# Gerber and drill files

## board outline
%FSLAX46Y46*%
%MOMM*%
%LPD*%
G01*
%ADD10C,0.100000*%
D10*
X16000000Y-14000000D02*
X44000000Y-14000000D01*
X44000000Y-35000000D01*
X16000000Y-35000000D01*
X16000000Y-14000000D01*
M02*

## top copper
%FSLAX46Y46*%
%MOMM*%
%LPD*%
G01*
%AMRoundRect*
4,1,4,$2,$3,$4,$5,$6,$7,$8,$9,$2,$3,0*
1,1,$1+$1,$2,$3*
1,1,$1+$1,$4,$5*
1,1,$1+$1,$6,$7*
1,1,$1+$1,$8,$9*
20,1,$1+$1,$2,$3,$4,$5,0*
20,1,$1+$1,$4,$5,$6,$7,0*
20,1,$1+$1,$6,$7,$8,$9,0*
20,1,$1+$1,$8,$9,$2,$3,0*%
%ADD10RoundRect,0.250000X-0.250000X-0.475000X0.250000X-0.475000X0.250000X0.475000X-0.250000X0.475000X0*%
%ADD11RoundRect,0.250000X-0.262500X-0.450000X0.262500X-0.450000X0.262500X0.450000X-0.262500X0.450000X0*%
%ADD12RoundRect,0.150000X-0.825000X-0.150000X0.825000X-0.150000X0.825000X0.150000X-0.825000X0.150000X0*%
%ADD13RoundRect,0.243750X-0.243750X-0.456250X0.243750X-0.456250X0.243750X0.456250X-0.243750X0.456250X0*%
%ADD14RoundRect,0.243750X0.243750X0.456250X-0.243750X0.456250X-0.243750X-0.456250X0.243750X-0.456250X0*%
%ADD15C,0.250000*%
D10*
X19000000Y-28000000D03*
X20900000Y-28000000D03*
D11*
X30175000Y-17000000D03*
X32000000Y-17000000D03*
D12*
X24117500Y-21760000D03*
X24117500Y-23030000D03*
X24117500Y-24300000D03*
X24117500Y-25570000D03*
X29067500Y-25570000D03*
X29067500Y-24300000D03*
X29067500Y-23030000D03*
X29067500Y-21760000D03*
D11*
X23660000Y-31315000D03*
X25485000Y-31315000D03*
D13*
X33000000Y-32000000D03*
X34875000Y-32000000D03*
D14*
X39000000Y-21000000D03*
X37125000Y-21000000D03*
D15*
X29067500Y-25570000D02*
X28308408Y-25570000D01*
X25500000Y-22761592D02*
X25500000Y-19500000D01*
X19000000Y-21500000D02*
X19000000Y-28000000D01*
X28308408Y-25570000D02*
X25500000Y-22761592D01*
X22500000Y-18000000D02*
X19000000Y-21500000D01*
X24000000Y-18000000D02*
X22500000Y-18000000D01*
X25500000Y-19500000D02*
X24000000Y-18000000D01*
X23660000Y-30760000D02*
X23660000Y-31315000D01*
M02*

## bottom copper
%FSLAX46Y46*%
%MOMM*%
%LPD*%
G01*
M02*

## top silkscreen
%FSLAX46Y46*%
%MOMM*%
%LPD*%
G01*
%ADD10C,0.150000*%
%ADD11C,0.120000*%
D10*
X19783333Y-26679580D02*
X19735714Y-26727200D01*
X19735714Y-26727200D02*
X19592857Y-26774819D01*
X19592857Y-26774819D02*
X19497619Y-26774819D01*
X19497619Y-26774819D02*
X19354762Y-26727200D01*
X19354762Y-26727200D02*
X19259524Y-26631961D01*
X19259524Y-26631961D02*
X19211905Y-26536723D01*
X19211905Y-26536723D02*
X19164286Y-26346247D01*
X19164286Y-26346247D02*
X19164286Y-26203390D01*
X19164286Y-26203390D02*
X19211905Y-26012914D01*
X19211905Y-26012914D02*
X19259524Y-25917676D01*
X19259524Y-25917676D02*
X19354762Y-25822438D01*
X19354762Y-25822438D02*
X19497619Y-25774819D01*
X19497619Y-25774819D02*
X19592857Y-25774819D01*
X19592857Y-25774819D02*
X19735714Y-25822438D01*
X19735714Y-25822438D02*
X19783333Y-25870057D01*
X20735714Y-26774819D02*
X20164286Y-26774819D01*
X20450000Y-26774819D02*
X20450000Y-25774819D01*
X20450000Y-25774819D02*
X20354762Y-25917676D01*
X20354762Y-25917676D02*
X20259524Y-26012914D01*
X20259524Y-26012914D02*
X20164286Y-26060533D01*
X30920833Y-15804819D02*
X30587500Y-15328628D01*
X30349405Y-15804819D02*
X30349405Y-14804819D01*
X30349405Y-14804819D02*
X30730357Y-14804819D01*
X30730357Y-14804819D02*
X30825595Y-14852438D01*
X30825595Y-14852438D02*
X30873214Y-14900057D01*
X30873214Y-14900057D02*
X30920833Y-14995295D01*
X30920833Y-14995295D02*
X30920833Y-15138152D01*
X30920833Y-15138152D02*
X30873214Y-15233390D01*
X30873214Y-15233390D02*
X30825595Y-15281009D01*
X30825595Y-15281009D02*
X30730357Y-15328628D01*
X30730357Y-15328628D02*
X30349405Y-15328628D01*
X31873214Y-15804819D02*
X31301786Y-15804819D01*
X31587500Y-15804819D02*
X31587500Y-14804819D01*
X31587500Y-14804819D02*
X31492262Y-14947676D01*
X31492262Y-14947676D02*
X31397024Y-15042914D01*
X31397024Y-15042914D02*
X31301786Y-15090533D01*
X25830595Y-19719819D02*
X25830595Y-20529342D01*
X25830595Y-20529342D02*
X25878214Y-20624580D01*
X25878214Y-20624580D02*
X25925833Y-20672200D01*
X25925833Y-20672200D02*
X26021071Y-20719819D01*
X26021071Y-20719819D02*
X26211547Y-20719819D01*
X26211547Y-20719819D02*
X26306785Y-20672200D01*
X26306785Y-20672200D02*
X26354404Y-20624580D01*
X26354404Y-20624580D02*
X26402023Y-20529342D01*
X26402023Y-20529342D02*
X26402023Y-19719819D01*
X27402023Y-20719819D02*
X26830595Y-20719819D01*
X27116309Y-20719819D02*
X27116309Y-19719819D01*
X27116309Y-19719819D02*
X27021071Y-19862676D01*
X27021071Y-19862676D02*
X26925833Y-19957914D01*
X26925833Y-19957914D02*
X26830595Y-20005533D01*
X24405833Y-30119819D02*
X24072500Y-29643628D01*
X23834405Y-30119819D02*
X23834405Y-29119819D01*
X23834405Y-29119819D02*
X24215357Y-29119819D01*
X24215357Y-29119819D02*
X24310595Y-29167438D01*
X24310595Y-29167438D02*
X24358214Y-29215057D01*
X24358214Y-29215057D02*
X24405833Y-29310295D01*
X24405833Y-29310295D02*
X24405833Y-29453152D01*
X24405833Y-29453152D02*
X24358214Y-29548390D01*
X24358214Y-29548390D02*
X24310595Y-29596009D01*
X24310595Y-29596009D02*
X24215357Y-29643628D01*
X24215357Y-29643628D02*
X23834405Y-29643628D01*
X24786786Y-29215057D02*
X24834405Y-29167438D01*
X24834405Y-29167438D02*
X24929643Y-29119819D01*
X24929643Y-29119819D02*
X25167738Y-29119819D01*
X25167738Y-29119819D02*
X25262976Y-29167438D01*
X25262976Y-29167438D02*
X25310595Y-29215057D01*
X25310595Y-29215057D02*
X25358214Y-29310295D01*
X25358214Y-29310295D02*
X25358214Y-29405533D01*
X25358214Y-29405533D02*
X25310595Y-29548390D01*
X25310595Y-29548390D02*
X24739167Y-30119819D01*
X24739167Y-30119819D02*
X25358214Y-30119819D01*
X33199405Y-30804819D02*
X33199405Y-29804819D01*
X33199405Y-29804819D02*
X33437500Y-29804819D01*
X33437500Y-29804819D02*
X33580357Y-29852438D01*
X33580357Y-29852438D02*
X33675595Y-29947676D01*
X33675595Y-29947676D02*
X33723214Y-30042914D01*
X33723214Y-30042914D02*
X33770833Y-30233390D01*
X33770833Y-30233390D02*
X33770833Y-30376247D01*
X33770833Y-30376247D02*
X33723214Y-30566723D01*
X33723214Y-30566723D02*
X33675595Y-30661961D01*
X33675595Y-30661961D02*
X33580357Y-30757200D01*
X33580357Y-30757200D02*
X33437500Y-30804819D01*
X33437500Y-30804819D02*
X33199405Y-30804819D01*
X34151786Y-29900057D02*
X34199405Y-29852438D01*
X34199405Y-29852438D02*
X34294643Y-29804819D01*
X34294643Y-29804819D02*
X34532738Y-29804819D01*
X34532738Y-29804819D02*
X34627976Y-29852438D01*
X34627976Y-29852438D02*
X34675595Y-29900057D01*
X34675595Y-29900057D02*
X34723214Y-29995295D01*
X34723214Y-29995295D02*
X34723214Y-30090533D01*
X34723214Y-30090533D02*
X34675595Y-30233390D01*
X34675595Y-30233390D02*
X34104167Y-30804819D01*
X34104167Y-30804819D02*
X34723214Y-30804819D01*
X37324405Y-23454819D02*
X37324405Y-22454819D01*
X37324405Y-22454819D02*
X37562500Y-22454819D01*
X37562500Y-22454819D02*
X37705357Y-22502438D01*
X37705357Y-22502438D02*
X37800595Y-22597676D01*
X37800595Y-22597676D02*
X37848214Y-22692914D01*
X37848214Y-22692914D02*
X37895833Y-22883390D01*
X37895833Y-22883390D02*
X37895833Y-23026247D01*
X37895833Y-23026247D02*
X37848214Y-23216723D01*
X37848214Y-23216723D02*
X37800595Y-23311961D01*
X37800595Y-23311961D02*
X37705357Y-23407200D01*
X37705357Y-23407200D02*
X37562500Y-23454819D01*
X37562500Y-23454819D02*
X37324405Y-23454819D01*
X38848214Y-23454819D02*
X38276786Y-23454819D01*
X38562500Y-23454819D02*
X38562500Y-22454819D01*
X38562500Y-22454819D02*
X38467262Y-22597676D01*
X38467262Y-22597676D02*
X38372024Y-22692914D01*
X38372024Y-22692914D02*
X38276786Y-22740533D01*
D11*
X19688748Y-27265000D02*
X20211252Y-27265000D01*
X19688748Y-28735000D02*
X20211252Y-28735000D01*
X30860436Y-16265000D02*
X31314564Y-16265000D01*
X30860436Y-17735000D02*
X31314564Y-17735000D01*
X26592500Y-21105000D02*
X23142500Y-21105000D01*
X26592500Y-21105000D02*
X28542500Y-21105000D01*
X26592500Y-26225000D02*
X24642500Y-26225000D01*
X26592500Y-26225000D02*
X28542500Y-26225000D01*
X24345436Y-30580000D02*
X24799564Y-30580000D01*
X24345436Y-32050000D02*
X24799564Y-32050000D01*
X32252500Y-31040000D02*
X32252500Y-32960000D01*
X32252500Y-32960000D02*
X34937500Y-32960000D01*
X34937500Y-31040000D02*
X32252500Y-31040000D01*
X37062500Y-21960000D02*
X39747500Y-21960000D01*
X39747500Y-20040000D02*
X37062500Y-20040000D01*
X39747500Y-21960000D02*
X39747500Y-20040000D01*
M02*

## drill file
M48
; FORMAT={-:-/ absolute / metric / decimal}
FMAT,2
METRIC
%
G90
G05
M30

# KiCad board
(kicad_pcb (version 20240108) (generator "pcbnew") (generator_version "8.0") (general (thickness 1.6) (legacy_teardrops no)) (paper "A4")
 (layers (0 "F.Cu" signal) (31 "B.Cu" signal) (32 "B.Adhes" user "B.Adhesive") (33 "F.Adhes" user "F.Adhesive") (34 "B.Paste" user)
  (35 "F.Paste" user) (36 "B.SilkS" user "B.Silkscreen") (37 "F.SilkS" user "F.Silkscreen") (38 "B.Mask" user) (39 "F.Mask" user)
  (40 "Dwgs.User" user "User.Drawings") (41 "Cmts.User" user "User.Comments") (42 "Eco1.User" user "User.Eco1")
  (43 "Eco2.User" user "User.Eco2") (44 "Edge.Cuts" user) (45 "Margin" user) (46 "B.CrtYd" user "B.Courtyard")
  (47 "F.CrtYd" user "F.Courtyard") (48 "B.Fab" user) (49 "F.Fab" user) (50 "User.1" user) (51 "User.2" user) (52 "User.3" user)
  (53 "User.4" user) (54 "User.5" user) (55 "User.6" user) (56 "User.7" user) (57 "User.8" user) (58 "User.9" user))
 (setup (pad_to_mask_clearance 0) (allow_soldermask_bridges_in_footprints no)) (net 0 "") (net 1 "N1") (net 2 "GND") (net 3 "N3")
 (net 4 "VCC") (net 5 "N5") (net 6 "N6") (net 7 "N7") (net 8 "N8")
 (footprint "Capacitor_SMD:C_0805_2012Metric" (layer "F.Cu") (at 19.95 28)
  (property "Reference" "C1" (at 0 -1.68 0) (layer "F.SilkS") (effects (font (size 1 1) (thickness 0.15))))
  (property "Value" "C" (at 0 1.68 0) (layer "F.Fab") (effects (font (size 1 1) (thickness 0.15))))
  (fp_line (start -0.261252 -0.735) (end 0.261252 -0.735) (stroke (width 0.12) (type solid)) (layer "F.SilkS"))
  (fp_line (start -0.261252 0.735) (end 0.261252 0.735) (stroke (width 0.12) (type solid)) (layer "F.SilkS"))
  (pad "1" smd roundrect (at -0.95 0) (size 1 1.45) (layers "F.Cu" "F.Paste" "F.Mask") (roundrect_rratio 0.25) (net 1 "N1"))
  (pad "2" smd roundrect (at 0.95 0) (size 1 1.45) (layers "F.Cu" "F.Paste" "F.Mask") (roundrect_rratio 0.25) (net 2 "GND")))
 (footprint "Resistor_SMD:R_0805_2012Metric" (layer "F.Cu") (at 31.0875 17)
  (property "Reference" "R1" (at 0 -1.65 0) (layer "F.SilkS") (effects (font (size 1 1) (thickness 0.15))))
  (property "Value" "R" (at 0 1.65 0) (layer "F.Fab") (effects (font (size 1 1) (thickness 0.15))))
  (fp_line (start -0.227064 -0.735) (end 0.227064 -0.735) (stroke (width 0.12) (type solid)) (layer "F.SilkS"))
  (fp_line (start -0.227064 0.735) (end 0.227064 0.735) (stroke (width 0.12) (type solid)) (layer "F.SilkS"))
  (pad "1" smd roundrect (at -0.9125 0) (size 1.025 1.4) (layers "F.Cu" "F.Paste" "F.Mask") (roundrect_rratio 0.243902) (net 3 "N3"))
  (pad "2" smd roundrect (at 0.9125 0) (size 1.025 1.4) (layers "F.Cu" "F.Paste" "F.Mask") (roundrect_rratio 0.243902) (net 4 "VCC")))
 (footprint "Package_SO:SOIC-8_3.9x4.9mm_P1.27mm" (layer "F.Cu") (at 26.5925 23.665)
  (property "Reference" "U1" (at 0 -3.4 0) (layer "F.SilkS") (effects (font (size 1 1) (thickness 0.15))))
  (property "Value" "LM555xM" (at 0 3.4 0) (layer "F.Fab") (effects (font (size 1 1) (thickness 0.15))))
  (fp_line (start 0 -2.56) (end -3.45 -2.56) (stroke (width 0.12) (type solid)) (layer "F.SilkS"))
  (fp_line (start 0 -2.56) (end 1.95 -2.56) (stroke (width 0.12) (type solid)) (layer "F.SilkS"))
  (fp_line (start 0 2.56) (end -1.95 2.56) (stroke (width 0.12) (type solid)) (layer "F.SilkS"))
  (fp_line (start 0 2.56) (end 1.95 2.56) (stroke (width 0.12) (type solid)) (layer "F.SilkS"))
  (pad "1" smd roundrect (at -2.475 -1.905) (size 1.95 0.6) (layers "F.Cu" "F.Paste" "F.Mask") (roundrect_rratio 0.25) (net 2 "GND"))
  (pad "2" smd roundrect (at -2.475 -0.635) (size 1.95 0.6) (layers "F.Cu" "F.Paste" "F.Mask") (roundrect_rratio 0.25) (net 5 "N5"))
  (pad "3" smd roundrect (at -2.475 0.635) (size 1.95 0.6) (layers "F.Cu" "F.Paste" "F.Mask") (roundrect_rratio 0.25) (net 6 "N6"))
  (pad "4" smd roundrect (at -2.475 1.905) (size 1.95 0.6) (layers "F.Cu" "F.Paste" "F.Mask") (roundrect_rratio 0.25) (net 4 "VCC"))
  (pad "5" smd roundrect (at 2.475 1.905) (size 1.95 0.6) (layers "F.Cu" "F.Paste" "F.Mask") (roundrect_rratio 0.25) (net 1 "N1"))
  (pad "6" smd roundrect (at 2.475 0.635) (size 1.95 0.6) (layers "F.Cu" "F.Paste" "F.Mask") (roundrect_rratio 0.25) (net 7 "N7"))
  (pad "7" smd roundrect (at 2.475 -0.635) (size 1.95 0.6) (layers "F.Cu" "F.Paste" "F.Mask") (roundrect_rratio 0.25) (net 7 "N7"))
  (pad "8" smd roundrect (at 2.475 -1.905) (size 1.95 0.6) (layers "F.Cu" "F.Paste" "F.Mask") (roundrect_rratio 0.25) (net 4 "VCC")))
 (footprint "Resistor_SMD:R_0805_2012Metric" (layer "F.Cu") (at 24.5725 31.315)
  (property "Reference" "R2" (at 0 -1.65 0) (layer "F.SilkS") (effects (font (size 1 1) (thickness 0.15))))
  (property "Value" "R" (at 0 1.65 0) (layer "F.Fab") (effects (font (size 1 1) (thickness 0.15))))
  (fp_line (start -0.227064 -0.735) (end 0.227064 -0.735) (stroke (width 0.12) (type solid)) (layer "F.SilkS"))
  (fp_line (start -0.227064 0.735) (end 0.227064 0.735) (stroke (width 0.12) (type solid)) (layer "F.SilkS"))
  (pad "1" smd roundrect (at -0.9125 0) (size 1.025 1.4) (layers "F.Cu" "F.Paste" "F.Mask") (roundrect_rratio 0.243902) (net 2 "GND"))
  (pad "2" smd roundrect (at 0.9125 0) (size 1.025 1.4) (layers "F.Cu" "F.Paste" "F.Mask") (roundrect_rratio 0.243902) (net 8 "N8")))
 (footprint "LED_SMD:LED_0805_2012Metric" (layer "F.Cu") (at 33.9375 32)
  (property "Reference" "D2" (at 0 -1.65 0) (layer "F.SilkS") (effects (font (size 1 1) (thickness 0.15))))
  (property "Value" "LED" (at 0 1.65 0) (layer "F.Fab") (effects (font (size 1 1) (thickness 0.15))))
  (fp_line (start -1.685 -0.96) (end -1.685 0.96) (stroke (width 0.12) (type solid)) (layer "F.SilkS"))
  (fp_line (start -1.685 0.96) (end 1 0.96) (stroke (width 0.12) (type solid)) (layer "F.SilkS"))
  (fp_line (start 1 -0.96) (end -1.685 -0.96) (stroke (width 0.12) (type solid)) (layer "F.SilkS"))
  (pad "1" smd roundrect (at -0.9375 0) (size 0.975 1.4) (layers "F.Cu" "F.Paste" "F.Mask") (roundrect_rratio 0.25) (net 8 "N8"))
  (pad "2" smd roundrect (at 0.9375 0) (size 0.975 1.4) (layers "F.Cu" "F.Paste" "F.Mask") (roundrect_rratio 0.25) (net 6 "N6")))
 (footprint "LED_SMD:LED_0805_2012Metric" (layer "F.Cu") (at 38.0625 21 180)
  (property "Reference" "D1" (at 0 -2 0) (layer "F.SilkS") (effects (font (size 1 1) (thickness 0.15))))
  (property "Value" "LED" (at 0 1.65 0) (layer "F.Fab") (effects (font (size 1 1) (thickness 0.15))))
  (fp_line (start 1 -0.96) (end -1.685 -0.96) (stroke (width 0.12) (type solid)) (layer "F.SilkS"))
  (fp_line (start -1.685 0.96) (end 1 0.96) (stroke (width 0.12) (type solid)) (layer "F.SilkS"))
  (fp_line (start -1.685 -0.96) (end -1.685 0.96) (stroke (width 0.12) (type solid)) (layer "F.SilkS"))
  (pad "1" smd roundrect (at -0.9375 0 180) (size 0.975 1.4) (layers "F.Cu" "F.Paste" "F.Mask") (roundrect_rratio 0.25) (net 6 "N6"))
  (pad "2" smd roundrect (at 0.9375 0 180) (size 0.975 1.4) (layers "F.Cu" "F.Paste" "F.Mask") (roundrect_rratio 0.25) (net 3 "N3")))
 (gr_rect (start 16 14) (end 44 35) (stroke (width 0.1) (type default)) (fill none) (layer "Edge.Cuts"))
 (segment (start 29.0675 25.57) (end 28.308408 25.57) (width 0.25) (layer "F.Cu") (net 1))
 (segment (start 25.5 22.761592) (end 25.5 19.5) (width 0.25) (layer "F.Cu") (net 1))
 (segment (start 19 21.5) (end 19 28) (width 0.25) (layer "F.Cu") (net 1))
 (segment (start 28.308408 25.57) (end 25.5 22.761592) (width 0.25) (layer "F.Cu") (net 1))
 (segment (start 22.5 18) (end 19 21.5) (width 0.25) (layer "F.Cu") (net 1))
 (segment (start 24 18) (end 22.5 18) (width 0.25) (layer "F.Cu") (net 1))
 (segment (start 25.5 19.5) (end 24 18) (width 0.25) (layer "F.Cu") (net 1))
 (segment (start 23.66 30.76) (end 23.66 31.315) (width 0.25) (layer "F.Cu") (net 2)))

